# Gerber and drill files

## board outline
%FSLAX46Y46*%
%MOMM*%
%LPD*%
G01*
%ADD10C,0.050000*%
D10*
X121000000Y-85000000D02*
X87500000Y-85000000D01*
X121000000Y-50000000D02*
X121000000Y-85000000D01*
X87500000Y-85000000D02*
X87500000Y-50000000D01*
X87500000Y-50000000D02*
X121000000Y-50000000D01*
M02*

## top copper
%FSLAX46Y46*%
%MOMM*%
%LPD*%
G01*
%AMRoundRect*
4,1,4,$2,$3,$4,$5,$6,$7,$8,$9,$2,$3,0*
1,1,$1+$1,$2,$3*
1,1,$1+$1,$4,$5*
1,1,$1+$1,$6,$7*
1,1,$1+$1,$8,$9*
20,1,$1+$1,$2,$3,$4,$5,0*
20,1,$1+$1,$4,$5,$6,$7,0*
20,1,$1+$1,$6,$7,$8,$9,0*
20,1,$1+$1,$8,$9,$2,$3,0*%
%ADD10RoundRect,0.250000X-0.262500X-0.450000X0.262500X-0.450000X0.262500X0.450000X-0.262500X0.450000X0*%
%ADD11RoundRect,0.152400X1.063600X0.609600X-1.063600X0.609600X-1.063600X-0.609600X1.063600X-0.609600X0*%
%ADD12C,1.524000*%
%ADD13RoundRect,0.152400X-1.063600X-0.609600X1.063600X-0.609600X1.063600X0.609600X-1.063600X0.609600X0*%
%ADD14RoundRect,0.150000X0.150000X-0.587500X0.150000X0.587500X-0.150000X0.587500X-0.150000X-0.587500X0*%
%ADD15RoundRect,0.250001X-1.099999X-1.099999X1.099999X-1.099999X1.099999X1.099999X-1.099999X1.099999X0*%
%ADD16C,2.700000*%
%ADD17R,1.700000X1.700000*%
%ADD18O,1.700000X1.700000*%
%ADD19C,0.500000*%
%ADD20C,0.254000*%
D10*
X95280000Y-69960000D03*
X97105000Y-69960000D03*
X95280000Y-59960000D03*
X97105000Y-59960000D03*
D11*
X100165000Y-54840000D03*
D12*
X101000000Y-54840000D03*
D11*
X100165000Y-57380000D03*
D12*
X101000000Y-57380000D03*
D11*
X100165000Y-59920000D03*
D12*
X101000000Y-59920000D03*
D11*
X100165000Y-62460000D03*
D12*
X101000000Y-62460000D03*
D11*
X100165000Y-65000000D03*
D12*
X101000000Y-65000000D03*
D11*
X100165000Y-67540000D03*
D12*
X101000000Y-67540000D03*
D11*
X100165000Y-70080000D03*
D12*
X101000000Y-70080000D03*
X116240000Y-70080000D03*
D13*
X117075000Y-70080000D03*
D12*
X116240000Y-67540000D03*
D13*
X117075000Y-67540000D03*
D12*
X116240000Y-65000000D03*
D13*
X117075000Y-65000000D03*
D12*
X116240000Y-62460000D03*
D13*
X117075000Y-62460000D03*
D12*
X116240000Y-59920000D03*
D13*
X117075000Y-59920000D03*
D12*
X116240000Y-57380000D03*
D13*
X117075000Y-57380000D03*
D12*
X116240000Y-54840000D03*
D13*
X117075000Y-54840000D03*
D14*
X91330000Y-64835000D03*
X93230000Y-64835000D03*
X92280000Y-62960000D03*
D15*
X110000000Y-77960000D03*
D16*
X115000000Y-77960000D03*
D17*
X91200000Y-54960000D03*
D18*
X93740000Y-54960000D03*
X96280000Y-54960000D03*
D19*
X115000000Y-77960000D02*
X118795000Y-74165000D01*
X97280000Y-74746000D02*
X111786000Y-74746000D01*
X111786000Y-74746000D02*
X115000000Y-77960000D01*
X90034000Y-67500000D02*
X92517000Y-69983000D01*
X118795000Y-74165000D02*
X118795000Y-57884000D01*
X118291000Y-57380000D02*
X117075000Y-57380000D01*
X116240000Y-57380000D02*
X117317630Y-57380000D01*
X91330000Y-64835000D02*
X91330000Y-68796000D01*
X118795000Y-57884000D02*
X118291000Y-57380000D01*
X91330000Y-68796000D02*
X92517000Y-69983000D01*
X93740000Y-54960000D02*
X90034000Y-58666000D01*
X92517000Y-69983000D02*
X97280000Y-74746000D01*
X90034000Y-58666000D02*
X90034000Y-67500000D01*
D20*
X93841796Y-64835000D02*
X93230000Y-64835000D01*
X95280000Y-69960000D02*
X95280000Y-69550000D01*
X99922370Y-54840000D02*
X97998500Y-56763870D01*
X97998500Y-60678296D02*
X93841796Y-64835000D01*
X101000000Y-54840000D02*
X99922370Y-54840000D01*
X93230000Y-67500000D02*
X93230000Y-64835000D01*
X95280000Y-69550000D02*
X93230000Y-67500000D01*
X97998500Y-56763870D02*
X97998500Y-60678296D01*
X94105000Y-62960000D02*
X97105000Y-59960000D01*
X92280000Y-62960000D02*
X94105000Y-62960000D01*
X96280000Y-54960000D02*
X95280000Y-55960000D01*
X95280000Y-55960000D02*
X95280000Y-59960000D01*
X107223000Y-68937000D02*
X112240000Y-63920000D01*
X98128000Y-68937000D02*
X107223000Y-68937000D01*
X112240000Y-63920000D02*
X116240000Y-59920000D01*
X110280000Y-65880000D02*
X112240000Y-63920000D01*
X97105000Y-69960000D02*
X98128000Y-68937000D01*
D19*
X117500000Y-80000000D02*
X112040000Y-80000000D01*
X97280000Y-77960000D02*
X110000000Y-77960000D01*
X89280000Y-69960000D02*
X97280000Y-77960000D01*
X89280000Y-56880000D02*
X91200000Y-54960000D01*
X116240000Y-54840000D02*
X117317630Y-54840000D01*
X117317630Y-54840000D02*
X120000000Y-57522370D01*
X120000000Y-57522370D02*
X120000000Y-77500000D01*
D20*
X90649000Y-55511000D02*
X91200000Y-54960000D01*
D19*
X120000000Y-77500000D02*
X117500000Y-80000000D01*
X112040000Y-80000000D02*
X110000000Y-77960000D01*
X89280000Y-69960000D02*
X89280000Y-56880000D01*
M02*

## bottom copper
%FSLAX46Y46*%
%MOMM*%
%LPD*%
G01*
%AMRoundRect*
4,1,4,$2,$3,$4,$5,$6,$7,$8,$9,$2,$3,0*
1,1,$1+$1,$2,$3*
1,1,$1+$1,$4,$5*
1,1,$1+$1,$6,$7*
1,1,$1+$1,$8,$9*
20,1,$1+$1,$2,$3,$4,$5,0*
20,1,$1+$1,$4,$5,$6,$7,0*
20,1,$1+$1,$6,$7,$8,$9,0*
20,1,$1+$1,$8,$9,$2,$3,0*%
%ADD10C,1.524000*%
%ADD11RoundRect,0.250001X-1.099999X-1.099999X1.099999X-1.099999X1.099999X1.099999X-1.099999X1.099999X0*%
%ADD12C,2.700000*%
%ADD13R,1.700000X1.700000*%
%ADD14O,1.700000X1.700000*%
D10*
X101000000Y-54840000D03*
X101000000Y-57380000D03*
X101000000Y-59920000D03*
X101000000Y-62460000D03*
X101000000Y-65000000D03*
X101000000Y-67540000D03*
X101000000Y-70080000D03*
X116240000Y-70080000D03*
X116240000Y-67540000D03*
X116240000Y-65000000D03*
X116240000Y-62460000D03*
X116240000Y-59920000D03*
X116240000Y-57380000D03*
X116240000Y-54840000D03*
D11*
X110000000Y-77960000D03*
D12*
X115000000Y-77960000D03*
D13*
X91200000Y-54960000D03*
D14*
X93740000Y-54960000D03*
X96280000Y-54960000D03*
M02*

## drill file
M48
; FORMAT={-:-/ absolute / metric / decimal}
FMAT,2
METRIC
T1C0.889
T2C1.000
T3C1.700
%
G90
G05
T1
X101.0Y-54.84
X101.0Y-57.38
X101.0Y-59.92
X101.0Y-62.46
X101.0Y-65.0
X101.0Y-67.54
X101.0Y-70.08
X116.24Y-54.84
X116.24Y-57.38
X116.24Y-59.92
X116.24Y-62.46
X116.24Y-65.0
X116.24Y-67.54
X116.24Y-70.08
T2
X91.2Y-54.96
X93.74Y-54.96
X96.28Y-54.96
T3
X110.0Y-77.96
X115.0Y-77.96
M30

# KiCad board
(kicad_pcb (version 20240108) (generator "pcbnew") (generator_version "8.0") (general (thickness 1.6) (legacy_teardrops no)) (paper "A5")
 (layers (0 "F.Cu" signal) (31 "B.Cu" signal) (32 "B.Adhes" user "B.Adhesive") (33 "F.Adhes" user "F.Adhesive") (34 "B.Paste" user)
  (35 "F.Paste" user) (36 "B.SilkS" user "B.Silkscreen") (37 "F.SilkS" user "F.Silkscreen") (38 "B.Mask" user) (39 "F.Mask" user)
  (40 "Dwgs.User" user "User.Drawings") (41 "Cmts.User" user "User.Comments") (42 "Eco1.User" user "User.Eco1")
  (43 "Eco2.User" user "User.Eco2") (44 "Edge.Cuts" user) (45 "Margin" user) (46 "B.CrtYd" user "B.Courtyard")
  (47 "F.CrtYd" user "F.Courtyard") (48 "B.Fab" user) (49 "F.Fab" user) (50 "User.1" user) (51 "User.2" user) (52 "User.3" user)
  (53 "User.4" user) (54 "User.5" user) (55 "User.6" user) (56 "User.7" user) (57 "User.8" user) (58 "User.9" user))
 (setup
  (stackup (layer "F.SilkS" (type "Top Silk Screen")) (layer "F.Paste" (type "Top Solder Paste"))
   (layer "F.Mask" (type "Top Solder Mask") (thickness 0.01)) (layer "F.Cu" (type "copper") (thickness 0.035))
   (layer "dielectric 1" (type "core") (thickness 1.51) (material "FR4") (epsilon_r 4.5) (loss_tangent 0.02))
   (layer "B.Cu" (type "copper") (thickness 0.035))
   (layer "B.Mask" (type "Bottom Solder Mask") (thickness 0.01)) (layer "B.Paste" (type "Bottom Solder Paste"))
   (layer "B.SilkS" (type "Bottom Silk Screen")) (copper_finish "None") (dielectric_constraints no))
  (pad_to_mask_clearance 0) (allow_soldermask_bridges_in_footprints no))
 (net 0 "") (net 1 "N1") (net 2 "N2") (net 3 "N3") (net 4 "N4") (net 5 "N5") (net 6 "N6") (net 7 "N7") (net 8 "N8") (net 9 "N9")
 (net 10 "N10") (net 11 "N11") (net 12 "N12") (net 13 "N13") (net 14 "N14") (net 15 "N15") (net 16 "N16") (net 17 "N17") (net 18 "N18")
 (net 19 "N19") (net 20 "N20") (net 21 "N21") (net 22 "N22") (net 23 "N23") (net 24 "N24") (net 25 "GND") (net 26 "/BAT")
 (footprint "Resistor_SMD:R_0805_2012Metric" (layer "F.Cu") (at 96.1925 69.96)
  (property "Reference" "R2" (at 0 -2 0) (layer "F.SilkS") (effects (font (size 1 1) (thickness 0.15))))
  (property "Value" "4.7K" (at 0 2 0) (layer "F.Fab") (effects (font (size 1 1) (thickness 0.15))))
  (pad "1" smd roundrect (at -0.9125 0) (size 1.025 1.4) (layers "F.Cu" "F.Paste" "F.Mask") (roundrect_rratio 0.243902) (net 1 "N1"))
  (pad "2" smd roundrect (at 0.9125 0) (size 1.025 1.4) (layers "F.Cu" "F.Paste" "F.Mask") (roundrect_rratio 0.243902) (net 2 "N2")))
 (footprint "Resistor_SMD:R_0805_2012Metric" (layer "F.Cu") (at 96.1925 59.96)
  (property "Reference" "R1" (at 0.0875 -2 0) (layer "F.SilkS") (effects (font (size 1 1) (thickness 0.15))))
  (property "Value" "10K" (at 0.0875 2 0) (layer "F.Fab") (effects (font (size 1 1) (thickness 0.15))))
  (pad "1" smd roundrect (at -0.9125 0) (size 1.025 1.4) (layers "F.Cu" "F.Paste" "F.Mask") (roundrect_rratio 0.243902) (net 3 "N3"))
  (pad "2" smd roundrect (at 0.9125 0) (size 1.025 1.4) (layers "F.Cu" "F.Paste" "F.Mask") (roundrect_rratio 0.243902) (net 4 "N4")))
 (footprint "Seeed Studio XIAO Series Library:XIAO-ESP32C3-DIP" (layer "F.Cu") (at 108.74 62.46)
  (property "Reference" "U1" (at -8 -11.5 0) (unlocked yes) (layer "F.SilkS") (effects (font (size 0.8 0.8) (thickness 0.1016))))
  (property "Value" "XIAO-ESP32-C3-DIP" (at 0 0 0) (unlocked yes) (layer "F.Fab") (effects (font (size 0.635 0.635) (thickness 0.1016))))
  (pad "1" smd roundrect (at -8.575 -7.62 180) (size 2.432 1.524) (layers "F.Cu" "F.Mask") (roundrect_rratio 0.1) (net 1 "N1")
   (thermal_bridge_angle 45))
  (pad "1" thru_hole circle (at -7.74 -7.62 180) (size 1.524 1.524) (drill 0.889) (layers "*.Cu" "*.Mask") (remove_unused_layers no)
   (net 1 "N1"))
  (pad "2" smd roundrect (at -8.575 -5.08 180) (size 2.432 1.524) (layers "F.Cu" "F.Mask") (roundrect_rratio 0.1) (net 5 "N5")
   (thermal_bridge_angle 45))
  (pad "2" thru_hole circle (at -7.74 -5.08 180) (size 1.524 1.524) (drill 0.889) (layers "*.Cu" "*.Mask") (remove_unused_layers no)
   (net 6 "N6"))
  (pad "3" smd roundrect (at -8.575 -2.54 180) (size 2.432 1.524) (layers "F.Cu" "F.Mask") (roundrect_rratio 0.1) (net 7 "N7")
   (thermal_bridge_angle 45))
  (pad "3" thru_hole circle (at -7.74 -2.54 180) (size 1.524 1.524) (drill 0.889) (layers "*.Cu" "*.Mask") (remove_unused_layers no)
   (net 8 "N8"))
  (pad "4" smd roundrect (at -8.575 0 180) (size 2.432 1.524) (layers "F.Cu" "F.Mask") (roundrect_rratio 0.1) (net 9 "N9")
   (thermal_bridge_angle 45))
  (pad "4" thru_hole circle (at -7.74 0 180) (size 1.524 1.524) (drill 0.889) (layers "*.Cu" "*.Mask") (remove_unused_layers no)
   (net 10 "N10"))
  (pad "5" smd roundrect (at -8.575 2.54 180) (size 2.432 1.524) (layers "F.Cu" "F.Mask") (roundrect_rratio 0.1) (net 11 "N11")
   (thermal_bridge_angle 45))
  (pad "5" thru_hole circle (at -7.74 2.54 180) (size 1.524 1.524) (drill 0.889) (layers "*.Cu" "*.Mask") (remove_unused_layers no)
   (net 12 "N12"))
  (pad "6" smd roundrect (at -8.575 5.08 180) (size 2.432 1.524) (layers "F.Cu" "F.Mask") (roundrect_rratio 0.1) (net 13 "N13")
   (thermal_bridge_angle 45))
  (pad "6" thru_hole circle (at -7.74 5.08 180) (size 1.524 1.524) (drill 0.889) (layers "*.Cu" "*.Mask") (remove_unused_layers no)
   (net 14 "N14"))
  (pad "7" smd roundrect (at -8.575 7.62 180) (size 2.432 1.524) (layers "F.Cu" "F.Mask") (roundrect_rratio 0.1) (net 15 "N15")
   (thermal_bridge_angle 45))
  (pad "7" thru_hole circle (at -7.74 7.62 180) (size 1.524 1.524) (drill 0.889) (layers "*.Cu" "*.Mask") (remove_unused_layers no)
   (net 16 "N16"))
  (pad "8" thru_hole circle (at 7.5 7.62) (size 1.524 1.524) (drill 0.889) (layers "*.Cu" "*.Mask") (remove_unused_layers no) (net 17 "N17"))
  (pad "8" smd roundrect (at 8.335 7.62) (size 2.432 1.524) (layers "F.Cu" "F.Mask") (roundrect_rratio 0.1) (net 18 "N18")
   (thermal_bridge_angle 45))
  (pad "9" thru_hole circle (at 7.5 5.08) (size 1.524 1.524) (drill 0.889) (layers "*.Cu" "*.Mask") (remove_unused_layers no) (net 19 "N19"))
  (pad "9" smd roundrect (at 8.335 5.08) (size 2.432 1.524) (layers "F.Cu" "F.Mask") (roundrect_rratio 0.1) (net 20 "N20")
   (thermal_bridge_angle 45))
  (pad "10" thru_hole circle (at 7.5 2.54) (size 1.524 1.524) (drill 0.889) (layers "*.Cu" "*.Mask") (remove_unused_layers no)
   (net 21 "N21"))
  (pad "10" smd roundrect (at 8.335 2.54) (size 2.432 1.524) (layers "F.Cu" "F.Mask") (roundrect_rratio 0.1) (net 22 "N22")
   (thermal_bridge_angle 45))
  (pad "11" thru_hole circle (at 7.5 0) (size 1.524 1.524) (drill 0.889) (layers "*.Cu" "*.Mask") (remove_unused_layers no) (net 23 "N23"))
  (pad "11" smd roundrect (at 8.335 0) (size 2.432 1.524) (layers "F.Cu" "F.Mask") (roundrect_rratio 0.1) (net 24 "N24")
   (thermal_bridge_angle 45))
  (pad "12" thru_hole circle (at 7.5 -2.54) (size 1.524 1.524) (drill 0.889) (layers "*.Cu" "*.Mask") (remove_unused_layers no) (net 2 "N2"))
  (pad "12" smd roundrect (at 8.335 -2.54) (size 2.432 1.524) (layers "F.Cu" "F.Mask") (roundrect_rratio 0.1) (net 2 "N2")
   (thermal_bridge_angle 45))
  (pad "13" thru_hole circle (at 7.5 -5.08) (size 1.524 1.524) (drill 0.889) (layers "*.Cu" "*.Mask") (remove_unused_layers no)
   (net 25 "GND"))
  (pad "13" smd roundrect (at 8.335 -5.08) (size 2.432 1.524) (layers "F.Cu" "F.Mask") (roundrect_rratio 0.1) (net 25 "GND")
   (thermal_bridge_angle 45))
  (pad "14" thru_hole circle (at 7.5 -7.62) (size 1.524 1.524) (drill 0.889) (layers "*.Cu" "*.Mask") (remove_unused_layers no)
   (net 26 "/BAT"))
  (pad "14" smd roundrect (at 8.335 -7.62) (size 2.432 1.524) (layers "F.Cu" "F.Mask") (roundrect_rratio 0.1) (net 26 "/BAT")
   (thermal_bridge_angle 45)))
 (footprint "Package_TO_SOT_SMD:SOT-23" (layer "F.Cu") (at 92.28 63.8975 90)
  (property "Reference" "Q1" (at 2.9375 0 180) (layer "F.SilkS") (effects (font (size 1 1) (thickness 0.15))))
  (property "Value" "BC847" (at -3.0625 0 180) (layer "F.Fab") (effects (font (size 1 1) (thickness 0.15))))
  (pad "1" smd roundrect (at -0.9375 -0.95 90) (size 1.475 0.6) (layers "F.Cu" "F.Paste" "F.Mask") (roundrect_rratio 0.25) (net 25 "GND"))
  (pad "2" smd roundrect (at -0.9375 0.95 90) (size 1.475 0.6) (layers "F.Cu" "F.Paste" "F.Mask") (roundrect_rratio 0.25) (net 1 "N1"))
  (pad "3" smd roundrect (at 0.9375 0 90) (size 1.475 0.6) (layers "F.Cu" "F.Paste" "F.Mask") (roundrect_rratio 0.25) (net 4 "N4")))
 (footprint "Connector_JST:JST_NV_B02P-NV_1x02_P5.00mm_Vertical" (layer "F.Cu") (at 110 77.96)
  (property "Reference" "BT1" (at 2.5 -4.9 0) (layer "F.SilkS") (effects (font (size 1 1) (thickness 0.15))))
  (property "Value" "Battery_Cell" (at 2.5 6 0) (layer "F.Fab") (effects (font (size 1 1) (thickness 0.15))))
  (pad "1" thru_hole roundrect (at 0 0) (size 2.7 2.7) (drill 1.7) (layers "*.Cu" "*.Mask") (remove_unused_layers no)
   (roundrect_rratio 0.092593) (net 26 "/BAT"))
  (pad "2" thru_hole circle (at 5 0) (size 2.7 2.7) (drill 1.7) (layers "*.Cu" "*.Mask") (remove_unused_layers no) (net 25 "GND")))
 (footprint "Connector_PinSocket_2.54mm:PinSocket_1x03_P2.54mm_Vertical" (layer "F.Cu") (at 91.2 54.96 90)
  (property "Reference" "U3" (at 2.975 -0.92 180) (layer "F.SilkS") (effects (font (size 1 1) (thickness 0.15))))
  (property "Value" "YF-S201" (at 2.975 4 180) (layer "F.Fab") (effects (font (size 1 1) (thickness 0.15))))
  (pad "1" thru_hole rect (at 0 0 90) (size 1.7 1.7) (drill 1) (layers "*.Cu" "*.Mask") (remove_unused_layers no) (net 26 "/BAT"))
  (pad "2" thru_hole oval (at 0 2.54 90) (size 1.7 1.7) (drill 1) (layers "*.Cu" "*.Mask") (remove_unused_layers no) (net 25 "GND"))
  (pad "3" thru_hole oval (at 0 5.08 90) (size 1.7 1.7) (drill 1) (layers "*.Cu" "*.Mask") (remove_unused_layers no) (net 3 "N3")))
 (gr_line (start 121 85) (end 87.5 85) (stroke (width 0.05) (type default)) (layer "Edge.Cuts"))
 (gr_line (start 121 50) (end 121 85) (stroke (width 0.05) (type default)) (layer "Edge.Cuts"))
 (gr_line (start 87.5 85) (end 87.5 50) (stroke (width 0.05) (type default)) (layer "Edge.Cuts"))
 (gr_line (start 87.5 50) (end 121 50) (stroke (width 0.05) (type default)) (layer "Edge.Cuts"))
 (segment (start 115 77.96) (end 118.795 74.165) (width 0.5) (layer "F.Cu") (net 25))
 (segment (start 97.28 74.746) (end 111.786 74.746) (width 0.5) (layer "F.Cu") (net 25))
 (segment (start 111.786 74.746) (end 115 77.96) (width 0.5) (layer "F.Cu") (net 25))
 (segment (start 90.034 67.5) (end 92.517 69.983) (width 0.5) (layer "F.Cu") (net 25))
 (segment (start 118.795 74.165) (end 118.795 57.884) (width 0.5) (layer "F.Cu") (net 25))
 (segment (start 118.291 57.38) (end 117.075 57.38) (width 0.5) (layer "F.Cu") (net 25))
 (segment (start 116.24 57.38) (end 117.31763 57.38) (width 0.5) (layer "F.Cu") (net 25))
 (segment (start 91.33 64.835) (end 91.33 68.796) (width 0.5) (layer "F.Cu") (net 25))
 (segment (start 118.795 57.884) (end 118.291 57.38) (width 0.5) (layer "F.Cu") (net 25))
 (segment (start 91.33 68.796) (end 92.517 69.983) (width 0.5) (layer "F.Cu") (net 25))
 (segment (start 93.74 54.96) (end 90.034 58.666) (width 0.5) (layer "F.Cu") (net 25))
 (segment (start 92.517 69.983) (end 97.28 74.746) (width 0.5) (layer "F.Cu") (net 25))
 (segment (start 90.034 58.666) (end 90.034 67.5) (width 0.5) (layer "F.Cu") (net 25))
 (segment (start 93.841796 64.835) (end 93.23 64.835) (width 0.254) (layer "F.Cu") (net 1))
 (segment (start 95.28 69.96) (end 95.28 69.55) (width 0.254) (layer "F.Cu") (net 1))
 (segment (start 99.92237 54.84) (end 97.9985 56.76387) (width 0.254) (layer "F.Cu") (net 1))
 (segment (start 97.9985 60.678296) (end 93.841796 64.835) (width 0.254) (layer "F.Cu") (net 1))
 (segment (start 101 54.84) (end 99.92237 54.84) (width 0.254) (layer "F.Cu") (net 1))
 (segment (start 93.23 67.5) (end 93.23 64.835) (width 0.254) (layer "F.Cu") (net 1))
 (segment (start 95.28 69.55) (end 93.23 67.5) (width 0.254) (layer "F.Cu") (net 1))
 (segment (start 97.9985 56.76387) (end 97.9985 60.678296) (width 0.254) (layer "F.Cu") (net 1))
 (segment (start 94.105 62.96) (end 97.105 59.96) (width 0.254) (layer "F.Cu") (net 4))
 (segment (start 92.28 62.96) (end 94.105 62.96) (width 0.254) (layer "F.Cu") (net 4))
 (segment (start 96.28 54.96) (end 95.28 55.96) (width 0.254) (layer "F.Cu") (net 3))
 (segment (start 95.28 55.96) (end 95.28 59.96) (width 0.254) (layer "F.Cu") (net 3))
 (segment (start 107.223 68.937) (end 112.24 63.92) (width 0.254) (layer "F.Cu") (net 2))
 (segment (start 98.128 68.937) (end 107.223 68.937) (width 0.254) (layer "F.Cu") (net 2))
 (segment (start 112.24 63.92) (end 116.24 59.92) (width 0.254) (layer "F.Cu") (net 2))
 (segment (start 110.28 65.88) (end 112.24 63.92) (width 0.254) (layer "F.Cu") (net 2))
 (segment (start 97.105 69.96) (end 98.128 68.937) (width 0.254) (layer "F.Cu") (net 2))
 (segment (start 117.5 80) (end 112.04 80) (width 0.5) (layer "F.Cu") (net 26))
 (segment (start 97.28 77.96) (end 110 77.96) (width 0.5) (layer "F.Cu") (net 26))
 (segment (start 89.28 69.96) (end 97.28 77.96) (width 0.5) (layer "F.Cu") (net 26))
 (segment (start 89.28 56.88) (end 91.2 54.96) (width 0.5) (layer "F.Cu") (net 26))
 (segment (start 116.24 54.84) (end 117.31763 54.84) (width 0.5) (layer "F.Cu") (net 26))
 (segment (start 117.31763 54.84) (end 120 57.52237) (width 0.5) (layer "F.Cu") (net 26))
 (segment (start 120 57.52237) (end 120 77.5) (width 0.5) (layer "F.Cu") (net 26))
 (segment (start 90.649 55.511) (end 91.2 54.96) (width 0.254) (layer "F.Cu") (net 26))
 (segment (start 120 77.5) (end 117.5 80) (width 0.5) (layer "F.Cu") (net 26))
 (segment (start 112.04 80) (end 110 77.96) (width 0.5) (layer "F.Cu") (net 26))
 (segment (start 89.28 69.96) (end 89.28 56.88) (width 0.5) (layer "F.Cu") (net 26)))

